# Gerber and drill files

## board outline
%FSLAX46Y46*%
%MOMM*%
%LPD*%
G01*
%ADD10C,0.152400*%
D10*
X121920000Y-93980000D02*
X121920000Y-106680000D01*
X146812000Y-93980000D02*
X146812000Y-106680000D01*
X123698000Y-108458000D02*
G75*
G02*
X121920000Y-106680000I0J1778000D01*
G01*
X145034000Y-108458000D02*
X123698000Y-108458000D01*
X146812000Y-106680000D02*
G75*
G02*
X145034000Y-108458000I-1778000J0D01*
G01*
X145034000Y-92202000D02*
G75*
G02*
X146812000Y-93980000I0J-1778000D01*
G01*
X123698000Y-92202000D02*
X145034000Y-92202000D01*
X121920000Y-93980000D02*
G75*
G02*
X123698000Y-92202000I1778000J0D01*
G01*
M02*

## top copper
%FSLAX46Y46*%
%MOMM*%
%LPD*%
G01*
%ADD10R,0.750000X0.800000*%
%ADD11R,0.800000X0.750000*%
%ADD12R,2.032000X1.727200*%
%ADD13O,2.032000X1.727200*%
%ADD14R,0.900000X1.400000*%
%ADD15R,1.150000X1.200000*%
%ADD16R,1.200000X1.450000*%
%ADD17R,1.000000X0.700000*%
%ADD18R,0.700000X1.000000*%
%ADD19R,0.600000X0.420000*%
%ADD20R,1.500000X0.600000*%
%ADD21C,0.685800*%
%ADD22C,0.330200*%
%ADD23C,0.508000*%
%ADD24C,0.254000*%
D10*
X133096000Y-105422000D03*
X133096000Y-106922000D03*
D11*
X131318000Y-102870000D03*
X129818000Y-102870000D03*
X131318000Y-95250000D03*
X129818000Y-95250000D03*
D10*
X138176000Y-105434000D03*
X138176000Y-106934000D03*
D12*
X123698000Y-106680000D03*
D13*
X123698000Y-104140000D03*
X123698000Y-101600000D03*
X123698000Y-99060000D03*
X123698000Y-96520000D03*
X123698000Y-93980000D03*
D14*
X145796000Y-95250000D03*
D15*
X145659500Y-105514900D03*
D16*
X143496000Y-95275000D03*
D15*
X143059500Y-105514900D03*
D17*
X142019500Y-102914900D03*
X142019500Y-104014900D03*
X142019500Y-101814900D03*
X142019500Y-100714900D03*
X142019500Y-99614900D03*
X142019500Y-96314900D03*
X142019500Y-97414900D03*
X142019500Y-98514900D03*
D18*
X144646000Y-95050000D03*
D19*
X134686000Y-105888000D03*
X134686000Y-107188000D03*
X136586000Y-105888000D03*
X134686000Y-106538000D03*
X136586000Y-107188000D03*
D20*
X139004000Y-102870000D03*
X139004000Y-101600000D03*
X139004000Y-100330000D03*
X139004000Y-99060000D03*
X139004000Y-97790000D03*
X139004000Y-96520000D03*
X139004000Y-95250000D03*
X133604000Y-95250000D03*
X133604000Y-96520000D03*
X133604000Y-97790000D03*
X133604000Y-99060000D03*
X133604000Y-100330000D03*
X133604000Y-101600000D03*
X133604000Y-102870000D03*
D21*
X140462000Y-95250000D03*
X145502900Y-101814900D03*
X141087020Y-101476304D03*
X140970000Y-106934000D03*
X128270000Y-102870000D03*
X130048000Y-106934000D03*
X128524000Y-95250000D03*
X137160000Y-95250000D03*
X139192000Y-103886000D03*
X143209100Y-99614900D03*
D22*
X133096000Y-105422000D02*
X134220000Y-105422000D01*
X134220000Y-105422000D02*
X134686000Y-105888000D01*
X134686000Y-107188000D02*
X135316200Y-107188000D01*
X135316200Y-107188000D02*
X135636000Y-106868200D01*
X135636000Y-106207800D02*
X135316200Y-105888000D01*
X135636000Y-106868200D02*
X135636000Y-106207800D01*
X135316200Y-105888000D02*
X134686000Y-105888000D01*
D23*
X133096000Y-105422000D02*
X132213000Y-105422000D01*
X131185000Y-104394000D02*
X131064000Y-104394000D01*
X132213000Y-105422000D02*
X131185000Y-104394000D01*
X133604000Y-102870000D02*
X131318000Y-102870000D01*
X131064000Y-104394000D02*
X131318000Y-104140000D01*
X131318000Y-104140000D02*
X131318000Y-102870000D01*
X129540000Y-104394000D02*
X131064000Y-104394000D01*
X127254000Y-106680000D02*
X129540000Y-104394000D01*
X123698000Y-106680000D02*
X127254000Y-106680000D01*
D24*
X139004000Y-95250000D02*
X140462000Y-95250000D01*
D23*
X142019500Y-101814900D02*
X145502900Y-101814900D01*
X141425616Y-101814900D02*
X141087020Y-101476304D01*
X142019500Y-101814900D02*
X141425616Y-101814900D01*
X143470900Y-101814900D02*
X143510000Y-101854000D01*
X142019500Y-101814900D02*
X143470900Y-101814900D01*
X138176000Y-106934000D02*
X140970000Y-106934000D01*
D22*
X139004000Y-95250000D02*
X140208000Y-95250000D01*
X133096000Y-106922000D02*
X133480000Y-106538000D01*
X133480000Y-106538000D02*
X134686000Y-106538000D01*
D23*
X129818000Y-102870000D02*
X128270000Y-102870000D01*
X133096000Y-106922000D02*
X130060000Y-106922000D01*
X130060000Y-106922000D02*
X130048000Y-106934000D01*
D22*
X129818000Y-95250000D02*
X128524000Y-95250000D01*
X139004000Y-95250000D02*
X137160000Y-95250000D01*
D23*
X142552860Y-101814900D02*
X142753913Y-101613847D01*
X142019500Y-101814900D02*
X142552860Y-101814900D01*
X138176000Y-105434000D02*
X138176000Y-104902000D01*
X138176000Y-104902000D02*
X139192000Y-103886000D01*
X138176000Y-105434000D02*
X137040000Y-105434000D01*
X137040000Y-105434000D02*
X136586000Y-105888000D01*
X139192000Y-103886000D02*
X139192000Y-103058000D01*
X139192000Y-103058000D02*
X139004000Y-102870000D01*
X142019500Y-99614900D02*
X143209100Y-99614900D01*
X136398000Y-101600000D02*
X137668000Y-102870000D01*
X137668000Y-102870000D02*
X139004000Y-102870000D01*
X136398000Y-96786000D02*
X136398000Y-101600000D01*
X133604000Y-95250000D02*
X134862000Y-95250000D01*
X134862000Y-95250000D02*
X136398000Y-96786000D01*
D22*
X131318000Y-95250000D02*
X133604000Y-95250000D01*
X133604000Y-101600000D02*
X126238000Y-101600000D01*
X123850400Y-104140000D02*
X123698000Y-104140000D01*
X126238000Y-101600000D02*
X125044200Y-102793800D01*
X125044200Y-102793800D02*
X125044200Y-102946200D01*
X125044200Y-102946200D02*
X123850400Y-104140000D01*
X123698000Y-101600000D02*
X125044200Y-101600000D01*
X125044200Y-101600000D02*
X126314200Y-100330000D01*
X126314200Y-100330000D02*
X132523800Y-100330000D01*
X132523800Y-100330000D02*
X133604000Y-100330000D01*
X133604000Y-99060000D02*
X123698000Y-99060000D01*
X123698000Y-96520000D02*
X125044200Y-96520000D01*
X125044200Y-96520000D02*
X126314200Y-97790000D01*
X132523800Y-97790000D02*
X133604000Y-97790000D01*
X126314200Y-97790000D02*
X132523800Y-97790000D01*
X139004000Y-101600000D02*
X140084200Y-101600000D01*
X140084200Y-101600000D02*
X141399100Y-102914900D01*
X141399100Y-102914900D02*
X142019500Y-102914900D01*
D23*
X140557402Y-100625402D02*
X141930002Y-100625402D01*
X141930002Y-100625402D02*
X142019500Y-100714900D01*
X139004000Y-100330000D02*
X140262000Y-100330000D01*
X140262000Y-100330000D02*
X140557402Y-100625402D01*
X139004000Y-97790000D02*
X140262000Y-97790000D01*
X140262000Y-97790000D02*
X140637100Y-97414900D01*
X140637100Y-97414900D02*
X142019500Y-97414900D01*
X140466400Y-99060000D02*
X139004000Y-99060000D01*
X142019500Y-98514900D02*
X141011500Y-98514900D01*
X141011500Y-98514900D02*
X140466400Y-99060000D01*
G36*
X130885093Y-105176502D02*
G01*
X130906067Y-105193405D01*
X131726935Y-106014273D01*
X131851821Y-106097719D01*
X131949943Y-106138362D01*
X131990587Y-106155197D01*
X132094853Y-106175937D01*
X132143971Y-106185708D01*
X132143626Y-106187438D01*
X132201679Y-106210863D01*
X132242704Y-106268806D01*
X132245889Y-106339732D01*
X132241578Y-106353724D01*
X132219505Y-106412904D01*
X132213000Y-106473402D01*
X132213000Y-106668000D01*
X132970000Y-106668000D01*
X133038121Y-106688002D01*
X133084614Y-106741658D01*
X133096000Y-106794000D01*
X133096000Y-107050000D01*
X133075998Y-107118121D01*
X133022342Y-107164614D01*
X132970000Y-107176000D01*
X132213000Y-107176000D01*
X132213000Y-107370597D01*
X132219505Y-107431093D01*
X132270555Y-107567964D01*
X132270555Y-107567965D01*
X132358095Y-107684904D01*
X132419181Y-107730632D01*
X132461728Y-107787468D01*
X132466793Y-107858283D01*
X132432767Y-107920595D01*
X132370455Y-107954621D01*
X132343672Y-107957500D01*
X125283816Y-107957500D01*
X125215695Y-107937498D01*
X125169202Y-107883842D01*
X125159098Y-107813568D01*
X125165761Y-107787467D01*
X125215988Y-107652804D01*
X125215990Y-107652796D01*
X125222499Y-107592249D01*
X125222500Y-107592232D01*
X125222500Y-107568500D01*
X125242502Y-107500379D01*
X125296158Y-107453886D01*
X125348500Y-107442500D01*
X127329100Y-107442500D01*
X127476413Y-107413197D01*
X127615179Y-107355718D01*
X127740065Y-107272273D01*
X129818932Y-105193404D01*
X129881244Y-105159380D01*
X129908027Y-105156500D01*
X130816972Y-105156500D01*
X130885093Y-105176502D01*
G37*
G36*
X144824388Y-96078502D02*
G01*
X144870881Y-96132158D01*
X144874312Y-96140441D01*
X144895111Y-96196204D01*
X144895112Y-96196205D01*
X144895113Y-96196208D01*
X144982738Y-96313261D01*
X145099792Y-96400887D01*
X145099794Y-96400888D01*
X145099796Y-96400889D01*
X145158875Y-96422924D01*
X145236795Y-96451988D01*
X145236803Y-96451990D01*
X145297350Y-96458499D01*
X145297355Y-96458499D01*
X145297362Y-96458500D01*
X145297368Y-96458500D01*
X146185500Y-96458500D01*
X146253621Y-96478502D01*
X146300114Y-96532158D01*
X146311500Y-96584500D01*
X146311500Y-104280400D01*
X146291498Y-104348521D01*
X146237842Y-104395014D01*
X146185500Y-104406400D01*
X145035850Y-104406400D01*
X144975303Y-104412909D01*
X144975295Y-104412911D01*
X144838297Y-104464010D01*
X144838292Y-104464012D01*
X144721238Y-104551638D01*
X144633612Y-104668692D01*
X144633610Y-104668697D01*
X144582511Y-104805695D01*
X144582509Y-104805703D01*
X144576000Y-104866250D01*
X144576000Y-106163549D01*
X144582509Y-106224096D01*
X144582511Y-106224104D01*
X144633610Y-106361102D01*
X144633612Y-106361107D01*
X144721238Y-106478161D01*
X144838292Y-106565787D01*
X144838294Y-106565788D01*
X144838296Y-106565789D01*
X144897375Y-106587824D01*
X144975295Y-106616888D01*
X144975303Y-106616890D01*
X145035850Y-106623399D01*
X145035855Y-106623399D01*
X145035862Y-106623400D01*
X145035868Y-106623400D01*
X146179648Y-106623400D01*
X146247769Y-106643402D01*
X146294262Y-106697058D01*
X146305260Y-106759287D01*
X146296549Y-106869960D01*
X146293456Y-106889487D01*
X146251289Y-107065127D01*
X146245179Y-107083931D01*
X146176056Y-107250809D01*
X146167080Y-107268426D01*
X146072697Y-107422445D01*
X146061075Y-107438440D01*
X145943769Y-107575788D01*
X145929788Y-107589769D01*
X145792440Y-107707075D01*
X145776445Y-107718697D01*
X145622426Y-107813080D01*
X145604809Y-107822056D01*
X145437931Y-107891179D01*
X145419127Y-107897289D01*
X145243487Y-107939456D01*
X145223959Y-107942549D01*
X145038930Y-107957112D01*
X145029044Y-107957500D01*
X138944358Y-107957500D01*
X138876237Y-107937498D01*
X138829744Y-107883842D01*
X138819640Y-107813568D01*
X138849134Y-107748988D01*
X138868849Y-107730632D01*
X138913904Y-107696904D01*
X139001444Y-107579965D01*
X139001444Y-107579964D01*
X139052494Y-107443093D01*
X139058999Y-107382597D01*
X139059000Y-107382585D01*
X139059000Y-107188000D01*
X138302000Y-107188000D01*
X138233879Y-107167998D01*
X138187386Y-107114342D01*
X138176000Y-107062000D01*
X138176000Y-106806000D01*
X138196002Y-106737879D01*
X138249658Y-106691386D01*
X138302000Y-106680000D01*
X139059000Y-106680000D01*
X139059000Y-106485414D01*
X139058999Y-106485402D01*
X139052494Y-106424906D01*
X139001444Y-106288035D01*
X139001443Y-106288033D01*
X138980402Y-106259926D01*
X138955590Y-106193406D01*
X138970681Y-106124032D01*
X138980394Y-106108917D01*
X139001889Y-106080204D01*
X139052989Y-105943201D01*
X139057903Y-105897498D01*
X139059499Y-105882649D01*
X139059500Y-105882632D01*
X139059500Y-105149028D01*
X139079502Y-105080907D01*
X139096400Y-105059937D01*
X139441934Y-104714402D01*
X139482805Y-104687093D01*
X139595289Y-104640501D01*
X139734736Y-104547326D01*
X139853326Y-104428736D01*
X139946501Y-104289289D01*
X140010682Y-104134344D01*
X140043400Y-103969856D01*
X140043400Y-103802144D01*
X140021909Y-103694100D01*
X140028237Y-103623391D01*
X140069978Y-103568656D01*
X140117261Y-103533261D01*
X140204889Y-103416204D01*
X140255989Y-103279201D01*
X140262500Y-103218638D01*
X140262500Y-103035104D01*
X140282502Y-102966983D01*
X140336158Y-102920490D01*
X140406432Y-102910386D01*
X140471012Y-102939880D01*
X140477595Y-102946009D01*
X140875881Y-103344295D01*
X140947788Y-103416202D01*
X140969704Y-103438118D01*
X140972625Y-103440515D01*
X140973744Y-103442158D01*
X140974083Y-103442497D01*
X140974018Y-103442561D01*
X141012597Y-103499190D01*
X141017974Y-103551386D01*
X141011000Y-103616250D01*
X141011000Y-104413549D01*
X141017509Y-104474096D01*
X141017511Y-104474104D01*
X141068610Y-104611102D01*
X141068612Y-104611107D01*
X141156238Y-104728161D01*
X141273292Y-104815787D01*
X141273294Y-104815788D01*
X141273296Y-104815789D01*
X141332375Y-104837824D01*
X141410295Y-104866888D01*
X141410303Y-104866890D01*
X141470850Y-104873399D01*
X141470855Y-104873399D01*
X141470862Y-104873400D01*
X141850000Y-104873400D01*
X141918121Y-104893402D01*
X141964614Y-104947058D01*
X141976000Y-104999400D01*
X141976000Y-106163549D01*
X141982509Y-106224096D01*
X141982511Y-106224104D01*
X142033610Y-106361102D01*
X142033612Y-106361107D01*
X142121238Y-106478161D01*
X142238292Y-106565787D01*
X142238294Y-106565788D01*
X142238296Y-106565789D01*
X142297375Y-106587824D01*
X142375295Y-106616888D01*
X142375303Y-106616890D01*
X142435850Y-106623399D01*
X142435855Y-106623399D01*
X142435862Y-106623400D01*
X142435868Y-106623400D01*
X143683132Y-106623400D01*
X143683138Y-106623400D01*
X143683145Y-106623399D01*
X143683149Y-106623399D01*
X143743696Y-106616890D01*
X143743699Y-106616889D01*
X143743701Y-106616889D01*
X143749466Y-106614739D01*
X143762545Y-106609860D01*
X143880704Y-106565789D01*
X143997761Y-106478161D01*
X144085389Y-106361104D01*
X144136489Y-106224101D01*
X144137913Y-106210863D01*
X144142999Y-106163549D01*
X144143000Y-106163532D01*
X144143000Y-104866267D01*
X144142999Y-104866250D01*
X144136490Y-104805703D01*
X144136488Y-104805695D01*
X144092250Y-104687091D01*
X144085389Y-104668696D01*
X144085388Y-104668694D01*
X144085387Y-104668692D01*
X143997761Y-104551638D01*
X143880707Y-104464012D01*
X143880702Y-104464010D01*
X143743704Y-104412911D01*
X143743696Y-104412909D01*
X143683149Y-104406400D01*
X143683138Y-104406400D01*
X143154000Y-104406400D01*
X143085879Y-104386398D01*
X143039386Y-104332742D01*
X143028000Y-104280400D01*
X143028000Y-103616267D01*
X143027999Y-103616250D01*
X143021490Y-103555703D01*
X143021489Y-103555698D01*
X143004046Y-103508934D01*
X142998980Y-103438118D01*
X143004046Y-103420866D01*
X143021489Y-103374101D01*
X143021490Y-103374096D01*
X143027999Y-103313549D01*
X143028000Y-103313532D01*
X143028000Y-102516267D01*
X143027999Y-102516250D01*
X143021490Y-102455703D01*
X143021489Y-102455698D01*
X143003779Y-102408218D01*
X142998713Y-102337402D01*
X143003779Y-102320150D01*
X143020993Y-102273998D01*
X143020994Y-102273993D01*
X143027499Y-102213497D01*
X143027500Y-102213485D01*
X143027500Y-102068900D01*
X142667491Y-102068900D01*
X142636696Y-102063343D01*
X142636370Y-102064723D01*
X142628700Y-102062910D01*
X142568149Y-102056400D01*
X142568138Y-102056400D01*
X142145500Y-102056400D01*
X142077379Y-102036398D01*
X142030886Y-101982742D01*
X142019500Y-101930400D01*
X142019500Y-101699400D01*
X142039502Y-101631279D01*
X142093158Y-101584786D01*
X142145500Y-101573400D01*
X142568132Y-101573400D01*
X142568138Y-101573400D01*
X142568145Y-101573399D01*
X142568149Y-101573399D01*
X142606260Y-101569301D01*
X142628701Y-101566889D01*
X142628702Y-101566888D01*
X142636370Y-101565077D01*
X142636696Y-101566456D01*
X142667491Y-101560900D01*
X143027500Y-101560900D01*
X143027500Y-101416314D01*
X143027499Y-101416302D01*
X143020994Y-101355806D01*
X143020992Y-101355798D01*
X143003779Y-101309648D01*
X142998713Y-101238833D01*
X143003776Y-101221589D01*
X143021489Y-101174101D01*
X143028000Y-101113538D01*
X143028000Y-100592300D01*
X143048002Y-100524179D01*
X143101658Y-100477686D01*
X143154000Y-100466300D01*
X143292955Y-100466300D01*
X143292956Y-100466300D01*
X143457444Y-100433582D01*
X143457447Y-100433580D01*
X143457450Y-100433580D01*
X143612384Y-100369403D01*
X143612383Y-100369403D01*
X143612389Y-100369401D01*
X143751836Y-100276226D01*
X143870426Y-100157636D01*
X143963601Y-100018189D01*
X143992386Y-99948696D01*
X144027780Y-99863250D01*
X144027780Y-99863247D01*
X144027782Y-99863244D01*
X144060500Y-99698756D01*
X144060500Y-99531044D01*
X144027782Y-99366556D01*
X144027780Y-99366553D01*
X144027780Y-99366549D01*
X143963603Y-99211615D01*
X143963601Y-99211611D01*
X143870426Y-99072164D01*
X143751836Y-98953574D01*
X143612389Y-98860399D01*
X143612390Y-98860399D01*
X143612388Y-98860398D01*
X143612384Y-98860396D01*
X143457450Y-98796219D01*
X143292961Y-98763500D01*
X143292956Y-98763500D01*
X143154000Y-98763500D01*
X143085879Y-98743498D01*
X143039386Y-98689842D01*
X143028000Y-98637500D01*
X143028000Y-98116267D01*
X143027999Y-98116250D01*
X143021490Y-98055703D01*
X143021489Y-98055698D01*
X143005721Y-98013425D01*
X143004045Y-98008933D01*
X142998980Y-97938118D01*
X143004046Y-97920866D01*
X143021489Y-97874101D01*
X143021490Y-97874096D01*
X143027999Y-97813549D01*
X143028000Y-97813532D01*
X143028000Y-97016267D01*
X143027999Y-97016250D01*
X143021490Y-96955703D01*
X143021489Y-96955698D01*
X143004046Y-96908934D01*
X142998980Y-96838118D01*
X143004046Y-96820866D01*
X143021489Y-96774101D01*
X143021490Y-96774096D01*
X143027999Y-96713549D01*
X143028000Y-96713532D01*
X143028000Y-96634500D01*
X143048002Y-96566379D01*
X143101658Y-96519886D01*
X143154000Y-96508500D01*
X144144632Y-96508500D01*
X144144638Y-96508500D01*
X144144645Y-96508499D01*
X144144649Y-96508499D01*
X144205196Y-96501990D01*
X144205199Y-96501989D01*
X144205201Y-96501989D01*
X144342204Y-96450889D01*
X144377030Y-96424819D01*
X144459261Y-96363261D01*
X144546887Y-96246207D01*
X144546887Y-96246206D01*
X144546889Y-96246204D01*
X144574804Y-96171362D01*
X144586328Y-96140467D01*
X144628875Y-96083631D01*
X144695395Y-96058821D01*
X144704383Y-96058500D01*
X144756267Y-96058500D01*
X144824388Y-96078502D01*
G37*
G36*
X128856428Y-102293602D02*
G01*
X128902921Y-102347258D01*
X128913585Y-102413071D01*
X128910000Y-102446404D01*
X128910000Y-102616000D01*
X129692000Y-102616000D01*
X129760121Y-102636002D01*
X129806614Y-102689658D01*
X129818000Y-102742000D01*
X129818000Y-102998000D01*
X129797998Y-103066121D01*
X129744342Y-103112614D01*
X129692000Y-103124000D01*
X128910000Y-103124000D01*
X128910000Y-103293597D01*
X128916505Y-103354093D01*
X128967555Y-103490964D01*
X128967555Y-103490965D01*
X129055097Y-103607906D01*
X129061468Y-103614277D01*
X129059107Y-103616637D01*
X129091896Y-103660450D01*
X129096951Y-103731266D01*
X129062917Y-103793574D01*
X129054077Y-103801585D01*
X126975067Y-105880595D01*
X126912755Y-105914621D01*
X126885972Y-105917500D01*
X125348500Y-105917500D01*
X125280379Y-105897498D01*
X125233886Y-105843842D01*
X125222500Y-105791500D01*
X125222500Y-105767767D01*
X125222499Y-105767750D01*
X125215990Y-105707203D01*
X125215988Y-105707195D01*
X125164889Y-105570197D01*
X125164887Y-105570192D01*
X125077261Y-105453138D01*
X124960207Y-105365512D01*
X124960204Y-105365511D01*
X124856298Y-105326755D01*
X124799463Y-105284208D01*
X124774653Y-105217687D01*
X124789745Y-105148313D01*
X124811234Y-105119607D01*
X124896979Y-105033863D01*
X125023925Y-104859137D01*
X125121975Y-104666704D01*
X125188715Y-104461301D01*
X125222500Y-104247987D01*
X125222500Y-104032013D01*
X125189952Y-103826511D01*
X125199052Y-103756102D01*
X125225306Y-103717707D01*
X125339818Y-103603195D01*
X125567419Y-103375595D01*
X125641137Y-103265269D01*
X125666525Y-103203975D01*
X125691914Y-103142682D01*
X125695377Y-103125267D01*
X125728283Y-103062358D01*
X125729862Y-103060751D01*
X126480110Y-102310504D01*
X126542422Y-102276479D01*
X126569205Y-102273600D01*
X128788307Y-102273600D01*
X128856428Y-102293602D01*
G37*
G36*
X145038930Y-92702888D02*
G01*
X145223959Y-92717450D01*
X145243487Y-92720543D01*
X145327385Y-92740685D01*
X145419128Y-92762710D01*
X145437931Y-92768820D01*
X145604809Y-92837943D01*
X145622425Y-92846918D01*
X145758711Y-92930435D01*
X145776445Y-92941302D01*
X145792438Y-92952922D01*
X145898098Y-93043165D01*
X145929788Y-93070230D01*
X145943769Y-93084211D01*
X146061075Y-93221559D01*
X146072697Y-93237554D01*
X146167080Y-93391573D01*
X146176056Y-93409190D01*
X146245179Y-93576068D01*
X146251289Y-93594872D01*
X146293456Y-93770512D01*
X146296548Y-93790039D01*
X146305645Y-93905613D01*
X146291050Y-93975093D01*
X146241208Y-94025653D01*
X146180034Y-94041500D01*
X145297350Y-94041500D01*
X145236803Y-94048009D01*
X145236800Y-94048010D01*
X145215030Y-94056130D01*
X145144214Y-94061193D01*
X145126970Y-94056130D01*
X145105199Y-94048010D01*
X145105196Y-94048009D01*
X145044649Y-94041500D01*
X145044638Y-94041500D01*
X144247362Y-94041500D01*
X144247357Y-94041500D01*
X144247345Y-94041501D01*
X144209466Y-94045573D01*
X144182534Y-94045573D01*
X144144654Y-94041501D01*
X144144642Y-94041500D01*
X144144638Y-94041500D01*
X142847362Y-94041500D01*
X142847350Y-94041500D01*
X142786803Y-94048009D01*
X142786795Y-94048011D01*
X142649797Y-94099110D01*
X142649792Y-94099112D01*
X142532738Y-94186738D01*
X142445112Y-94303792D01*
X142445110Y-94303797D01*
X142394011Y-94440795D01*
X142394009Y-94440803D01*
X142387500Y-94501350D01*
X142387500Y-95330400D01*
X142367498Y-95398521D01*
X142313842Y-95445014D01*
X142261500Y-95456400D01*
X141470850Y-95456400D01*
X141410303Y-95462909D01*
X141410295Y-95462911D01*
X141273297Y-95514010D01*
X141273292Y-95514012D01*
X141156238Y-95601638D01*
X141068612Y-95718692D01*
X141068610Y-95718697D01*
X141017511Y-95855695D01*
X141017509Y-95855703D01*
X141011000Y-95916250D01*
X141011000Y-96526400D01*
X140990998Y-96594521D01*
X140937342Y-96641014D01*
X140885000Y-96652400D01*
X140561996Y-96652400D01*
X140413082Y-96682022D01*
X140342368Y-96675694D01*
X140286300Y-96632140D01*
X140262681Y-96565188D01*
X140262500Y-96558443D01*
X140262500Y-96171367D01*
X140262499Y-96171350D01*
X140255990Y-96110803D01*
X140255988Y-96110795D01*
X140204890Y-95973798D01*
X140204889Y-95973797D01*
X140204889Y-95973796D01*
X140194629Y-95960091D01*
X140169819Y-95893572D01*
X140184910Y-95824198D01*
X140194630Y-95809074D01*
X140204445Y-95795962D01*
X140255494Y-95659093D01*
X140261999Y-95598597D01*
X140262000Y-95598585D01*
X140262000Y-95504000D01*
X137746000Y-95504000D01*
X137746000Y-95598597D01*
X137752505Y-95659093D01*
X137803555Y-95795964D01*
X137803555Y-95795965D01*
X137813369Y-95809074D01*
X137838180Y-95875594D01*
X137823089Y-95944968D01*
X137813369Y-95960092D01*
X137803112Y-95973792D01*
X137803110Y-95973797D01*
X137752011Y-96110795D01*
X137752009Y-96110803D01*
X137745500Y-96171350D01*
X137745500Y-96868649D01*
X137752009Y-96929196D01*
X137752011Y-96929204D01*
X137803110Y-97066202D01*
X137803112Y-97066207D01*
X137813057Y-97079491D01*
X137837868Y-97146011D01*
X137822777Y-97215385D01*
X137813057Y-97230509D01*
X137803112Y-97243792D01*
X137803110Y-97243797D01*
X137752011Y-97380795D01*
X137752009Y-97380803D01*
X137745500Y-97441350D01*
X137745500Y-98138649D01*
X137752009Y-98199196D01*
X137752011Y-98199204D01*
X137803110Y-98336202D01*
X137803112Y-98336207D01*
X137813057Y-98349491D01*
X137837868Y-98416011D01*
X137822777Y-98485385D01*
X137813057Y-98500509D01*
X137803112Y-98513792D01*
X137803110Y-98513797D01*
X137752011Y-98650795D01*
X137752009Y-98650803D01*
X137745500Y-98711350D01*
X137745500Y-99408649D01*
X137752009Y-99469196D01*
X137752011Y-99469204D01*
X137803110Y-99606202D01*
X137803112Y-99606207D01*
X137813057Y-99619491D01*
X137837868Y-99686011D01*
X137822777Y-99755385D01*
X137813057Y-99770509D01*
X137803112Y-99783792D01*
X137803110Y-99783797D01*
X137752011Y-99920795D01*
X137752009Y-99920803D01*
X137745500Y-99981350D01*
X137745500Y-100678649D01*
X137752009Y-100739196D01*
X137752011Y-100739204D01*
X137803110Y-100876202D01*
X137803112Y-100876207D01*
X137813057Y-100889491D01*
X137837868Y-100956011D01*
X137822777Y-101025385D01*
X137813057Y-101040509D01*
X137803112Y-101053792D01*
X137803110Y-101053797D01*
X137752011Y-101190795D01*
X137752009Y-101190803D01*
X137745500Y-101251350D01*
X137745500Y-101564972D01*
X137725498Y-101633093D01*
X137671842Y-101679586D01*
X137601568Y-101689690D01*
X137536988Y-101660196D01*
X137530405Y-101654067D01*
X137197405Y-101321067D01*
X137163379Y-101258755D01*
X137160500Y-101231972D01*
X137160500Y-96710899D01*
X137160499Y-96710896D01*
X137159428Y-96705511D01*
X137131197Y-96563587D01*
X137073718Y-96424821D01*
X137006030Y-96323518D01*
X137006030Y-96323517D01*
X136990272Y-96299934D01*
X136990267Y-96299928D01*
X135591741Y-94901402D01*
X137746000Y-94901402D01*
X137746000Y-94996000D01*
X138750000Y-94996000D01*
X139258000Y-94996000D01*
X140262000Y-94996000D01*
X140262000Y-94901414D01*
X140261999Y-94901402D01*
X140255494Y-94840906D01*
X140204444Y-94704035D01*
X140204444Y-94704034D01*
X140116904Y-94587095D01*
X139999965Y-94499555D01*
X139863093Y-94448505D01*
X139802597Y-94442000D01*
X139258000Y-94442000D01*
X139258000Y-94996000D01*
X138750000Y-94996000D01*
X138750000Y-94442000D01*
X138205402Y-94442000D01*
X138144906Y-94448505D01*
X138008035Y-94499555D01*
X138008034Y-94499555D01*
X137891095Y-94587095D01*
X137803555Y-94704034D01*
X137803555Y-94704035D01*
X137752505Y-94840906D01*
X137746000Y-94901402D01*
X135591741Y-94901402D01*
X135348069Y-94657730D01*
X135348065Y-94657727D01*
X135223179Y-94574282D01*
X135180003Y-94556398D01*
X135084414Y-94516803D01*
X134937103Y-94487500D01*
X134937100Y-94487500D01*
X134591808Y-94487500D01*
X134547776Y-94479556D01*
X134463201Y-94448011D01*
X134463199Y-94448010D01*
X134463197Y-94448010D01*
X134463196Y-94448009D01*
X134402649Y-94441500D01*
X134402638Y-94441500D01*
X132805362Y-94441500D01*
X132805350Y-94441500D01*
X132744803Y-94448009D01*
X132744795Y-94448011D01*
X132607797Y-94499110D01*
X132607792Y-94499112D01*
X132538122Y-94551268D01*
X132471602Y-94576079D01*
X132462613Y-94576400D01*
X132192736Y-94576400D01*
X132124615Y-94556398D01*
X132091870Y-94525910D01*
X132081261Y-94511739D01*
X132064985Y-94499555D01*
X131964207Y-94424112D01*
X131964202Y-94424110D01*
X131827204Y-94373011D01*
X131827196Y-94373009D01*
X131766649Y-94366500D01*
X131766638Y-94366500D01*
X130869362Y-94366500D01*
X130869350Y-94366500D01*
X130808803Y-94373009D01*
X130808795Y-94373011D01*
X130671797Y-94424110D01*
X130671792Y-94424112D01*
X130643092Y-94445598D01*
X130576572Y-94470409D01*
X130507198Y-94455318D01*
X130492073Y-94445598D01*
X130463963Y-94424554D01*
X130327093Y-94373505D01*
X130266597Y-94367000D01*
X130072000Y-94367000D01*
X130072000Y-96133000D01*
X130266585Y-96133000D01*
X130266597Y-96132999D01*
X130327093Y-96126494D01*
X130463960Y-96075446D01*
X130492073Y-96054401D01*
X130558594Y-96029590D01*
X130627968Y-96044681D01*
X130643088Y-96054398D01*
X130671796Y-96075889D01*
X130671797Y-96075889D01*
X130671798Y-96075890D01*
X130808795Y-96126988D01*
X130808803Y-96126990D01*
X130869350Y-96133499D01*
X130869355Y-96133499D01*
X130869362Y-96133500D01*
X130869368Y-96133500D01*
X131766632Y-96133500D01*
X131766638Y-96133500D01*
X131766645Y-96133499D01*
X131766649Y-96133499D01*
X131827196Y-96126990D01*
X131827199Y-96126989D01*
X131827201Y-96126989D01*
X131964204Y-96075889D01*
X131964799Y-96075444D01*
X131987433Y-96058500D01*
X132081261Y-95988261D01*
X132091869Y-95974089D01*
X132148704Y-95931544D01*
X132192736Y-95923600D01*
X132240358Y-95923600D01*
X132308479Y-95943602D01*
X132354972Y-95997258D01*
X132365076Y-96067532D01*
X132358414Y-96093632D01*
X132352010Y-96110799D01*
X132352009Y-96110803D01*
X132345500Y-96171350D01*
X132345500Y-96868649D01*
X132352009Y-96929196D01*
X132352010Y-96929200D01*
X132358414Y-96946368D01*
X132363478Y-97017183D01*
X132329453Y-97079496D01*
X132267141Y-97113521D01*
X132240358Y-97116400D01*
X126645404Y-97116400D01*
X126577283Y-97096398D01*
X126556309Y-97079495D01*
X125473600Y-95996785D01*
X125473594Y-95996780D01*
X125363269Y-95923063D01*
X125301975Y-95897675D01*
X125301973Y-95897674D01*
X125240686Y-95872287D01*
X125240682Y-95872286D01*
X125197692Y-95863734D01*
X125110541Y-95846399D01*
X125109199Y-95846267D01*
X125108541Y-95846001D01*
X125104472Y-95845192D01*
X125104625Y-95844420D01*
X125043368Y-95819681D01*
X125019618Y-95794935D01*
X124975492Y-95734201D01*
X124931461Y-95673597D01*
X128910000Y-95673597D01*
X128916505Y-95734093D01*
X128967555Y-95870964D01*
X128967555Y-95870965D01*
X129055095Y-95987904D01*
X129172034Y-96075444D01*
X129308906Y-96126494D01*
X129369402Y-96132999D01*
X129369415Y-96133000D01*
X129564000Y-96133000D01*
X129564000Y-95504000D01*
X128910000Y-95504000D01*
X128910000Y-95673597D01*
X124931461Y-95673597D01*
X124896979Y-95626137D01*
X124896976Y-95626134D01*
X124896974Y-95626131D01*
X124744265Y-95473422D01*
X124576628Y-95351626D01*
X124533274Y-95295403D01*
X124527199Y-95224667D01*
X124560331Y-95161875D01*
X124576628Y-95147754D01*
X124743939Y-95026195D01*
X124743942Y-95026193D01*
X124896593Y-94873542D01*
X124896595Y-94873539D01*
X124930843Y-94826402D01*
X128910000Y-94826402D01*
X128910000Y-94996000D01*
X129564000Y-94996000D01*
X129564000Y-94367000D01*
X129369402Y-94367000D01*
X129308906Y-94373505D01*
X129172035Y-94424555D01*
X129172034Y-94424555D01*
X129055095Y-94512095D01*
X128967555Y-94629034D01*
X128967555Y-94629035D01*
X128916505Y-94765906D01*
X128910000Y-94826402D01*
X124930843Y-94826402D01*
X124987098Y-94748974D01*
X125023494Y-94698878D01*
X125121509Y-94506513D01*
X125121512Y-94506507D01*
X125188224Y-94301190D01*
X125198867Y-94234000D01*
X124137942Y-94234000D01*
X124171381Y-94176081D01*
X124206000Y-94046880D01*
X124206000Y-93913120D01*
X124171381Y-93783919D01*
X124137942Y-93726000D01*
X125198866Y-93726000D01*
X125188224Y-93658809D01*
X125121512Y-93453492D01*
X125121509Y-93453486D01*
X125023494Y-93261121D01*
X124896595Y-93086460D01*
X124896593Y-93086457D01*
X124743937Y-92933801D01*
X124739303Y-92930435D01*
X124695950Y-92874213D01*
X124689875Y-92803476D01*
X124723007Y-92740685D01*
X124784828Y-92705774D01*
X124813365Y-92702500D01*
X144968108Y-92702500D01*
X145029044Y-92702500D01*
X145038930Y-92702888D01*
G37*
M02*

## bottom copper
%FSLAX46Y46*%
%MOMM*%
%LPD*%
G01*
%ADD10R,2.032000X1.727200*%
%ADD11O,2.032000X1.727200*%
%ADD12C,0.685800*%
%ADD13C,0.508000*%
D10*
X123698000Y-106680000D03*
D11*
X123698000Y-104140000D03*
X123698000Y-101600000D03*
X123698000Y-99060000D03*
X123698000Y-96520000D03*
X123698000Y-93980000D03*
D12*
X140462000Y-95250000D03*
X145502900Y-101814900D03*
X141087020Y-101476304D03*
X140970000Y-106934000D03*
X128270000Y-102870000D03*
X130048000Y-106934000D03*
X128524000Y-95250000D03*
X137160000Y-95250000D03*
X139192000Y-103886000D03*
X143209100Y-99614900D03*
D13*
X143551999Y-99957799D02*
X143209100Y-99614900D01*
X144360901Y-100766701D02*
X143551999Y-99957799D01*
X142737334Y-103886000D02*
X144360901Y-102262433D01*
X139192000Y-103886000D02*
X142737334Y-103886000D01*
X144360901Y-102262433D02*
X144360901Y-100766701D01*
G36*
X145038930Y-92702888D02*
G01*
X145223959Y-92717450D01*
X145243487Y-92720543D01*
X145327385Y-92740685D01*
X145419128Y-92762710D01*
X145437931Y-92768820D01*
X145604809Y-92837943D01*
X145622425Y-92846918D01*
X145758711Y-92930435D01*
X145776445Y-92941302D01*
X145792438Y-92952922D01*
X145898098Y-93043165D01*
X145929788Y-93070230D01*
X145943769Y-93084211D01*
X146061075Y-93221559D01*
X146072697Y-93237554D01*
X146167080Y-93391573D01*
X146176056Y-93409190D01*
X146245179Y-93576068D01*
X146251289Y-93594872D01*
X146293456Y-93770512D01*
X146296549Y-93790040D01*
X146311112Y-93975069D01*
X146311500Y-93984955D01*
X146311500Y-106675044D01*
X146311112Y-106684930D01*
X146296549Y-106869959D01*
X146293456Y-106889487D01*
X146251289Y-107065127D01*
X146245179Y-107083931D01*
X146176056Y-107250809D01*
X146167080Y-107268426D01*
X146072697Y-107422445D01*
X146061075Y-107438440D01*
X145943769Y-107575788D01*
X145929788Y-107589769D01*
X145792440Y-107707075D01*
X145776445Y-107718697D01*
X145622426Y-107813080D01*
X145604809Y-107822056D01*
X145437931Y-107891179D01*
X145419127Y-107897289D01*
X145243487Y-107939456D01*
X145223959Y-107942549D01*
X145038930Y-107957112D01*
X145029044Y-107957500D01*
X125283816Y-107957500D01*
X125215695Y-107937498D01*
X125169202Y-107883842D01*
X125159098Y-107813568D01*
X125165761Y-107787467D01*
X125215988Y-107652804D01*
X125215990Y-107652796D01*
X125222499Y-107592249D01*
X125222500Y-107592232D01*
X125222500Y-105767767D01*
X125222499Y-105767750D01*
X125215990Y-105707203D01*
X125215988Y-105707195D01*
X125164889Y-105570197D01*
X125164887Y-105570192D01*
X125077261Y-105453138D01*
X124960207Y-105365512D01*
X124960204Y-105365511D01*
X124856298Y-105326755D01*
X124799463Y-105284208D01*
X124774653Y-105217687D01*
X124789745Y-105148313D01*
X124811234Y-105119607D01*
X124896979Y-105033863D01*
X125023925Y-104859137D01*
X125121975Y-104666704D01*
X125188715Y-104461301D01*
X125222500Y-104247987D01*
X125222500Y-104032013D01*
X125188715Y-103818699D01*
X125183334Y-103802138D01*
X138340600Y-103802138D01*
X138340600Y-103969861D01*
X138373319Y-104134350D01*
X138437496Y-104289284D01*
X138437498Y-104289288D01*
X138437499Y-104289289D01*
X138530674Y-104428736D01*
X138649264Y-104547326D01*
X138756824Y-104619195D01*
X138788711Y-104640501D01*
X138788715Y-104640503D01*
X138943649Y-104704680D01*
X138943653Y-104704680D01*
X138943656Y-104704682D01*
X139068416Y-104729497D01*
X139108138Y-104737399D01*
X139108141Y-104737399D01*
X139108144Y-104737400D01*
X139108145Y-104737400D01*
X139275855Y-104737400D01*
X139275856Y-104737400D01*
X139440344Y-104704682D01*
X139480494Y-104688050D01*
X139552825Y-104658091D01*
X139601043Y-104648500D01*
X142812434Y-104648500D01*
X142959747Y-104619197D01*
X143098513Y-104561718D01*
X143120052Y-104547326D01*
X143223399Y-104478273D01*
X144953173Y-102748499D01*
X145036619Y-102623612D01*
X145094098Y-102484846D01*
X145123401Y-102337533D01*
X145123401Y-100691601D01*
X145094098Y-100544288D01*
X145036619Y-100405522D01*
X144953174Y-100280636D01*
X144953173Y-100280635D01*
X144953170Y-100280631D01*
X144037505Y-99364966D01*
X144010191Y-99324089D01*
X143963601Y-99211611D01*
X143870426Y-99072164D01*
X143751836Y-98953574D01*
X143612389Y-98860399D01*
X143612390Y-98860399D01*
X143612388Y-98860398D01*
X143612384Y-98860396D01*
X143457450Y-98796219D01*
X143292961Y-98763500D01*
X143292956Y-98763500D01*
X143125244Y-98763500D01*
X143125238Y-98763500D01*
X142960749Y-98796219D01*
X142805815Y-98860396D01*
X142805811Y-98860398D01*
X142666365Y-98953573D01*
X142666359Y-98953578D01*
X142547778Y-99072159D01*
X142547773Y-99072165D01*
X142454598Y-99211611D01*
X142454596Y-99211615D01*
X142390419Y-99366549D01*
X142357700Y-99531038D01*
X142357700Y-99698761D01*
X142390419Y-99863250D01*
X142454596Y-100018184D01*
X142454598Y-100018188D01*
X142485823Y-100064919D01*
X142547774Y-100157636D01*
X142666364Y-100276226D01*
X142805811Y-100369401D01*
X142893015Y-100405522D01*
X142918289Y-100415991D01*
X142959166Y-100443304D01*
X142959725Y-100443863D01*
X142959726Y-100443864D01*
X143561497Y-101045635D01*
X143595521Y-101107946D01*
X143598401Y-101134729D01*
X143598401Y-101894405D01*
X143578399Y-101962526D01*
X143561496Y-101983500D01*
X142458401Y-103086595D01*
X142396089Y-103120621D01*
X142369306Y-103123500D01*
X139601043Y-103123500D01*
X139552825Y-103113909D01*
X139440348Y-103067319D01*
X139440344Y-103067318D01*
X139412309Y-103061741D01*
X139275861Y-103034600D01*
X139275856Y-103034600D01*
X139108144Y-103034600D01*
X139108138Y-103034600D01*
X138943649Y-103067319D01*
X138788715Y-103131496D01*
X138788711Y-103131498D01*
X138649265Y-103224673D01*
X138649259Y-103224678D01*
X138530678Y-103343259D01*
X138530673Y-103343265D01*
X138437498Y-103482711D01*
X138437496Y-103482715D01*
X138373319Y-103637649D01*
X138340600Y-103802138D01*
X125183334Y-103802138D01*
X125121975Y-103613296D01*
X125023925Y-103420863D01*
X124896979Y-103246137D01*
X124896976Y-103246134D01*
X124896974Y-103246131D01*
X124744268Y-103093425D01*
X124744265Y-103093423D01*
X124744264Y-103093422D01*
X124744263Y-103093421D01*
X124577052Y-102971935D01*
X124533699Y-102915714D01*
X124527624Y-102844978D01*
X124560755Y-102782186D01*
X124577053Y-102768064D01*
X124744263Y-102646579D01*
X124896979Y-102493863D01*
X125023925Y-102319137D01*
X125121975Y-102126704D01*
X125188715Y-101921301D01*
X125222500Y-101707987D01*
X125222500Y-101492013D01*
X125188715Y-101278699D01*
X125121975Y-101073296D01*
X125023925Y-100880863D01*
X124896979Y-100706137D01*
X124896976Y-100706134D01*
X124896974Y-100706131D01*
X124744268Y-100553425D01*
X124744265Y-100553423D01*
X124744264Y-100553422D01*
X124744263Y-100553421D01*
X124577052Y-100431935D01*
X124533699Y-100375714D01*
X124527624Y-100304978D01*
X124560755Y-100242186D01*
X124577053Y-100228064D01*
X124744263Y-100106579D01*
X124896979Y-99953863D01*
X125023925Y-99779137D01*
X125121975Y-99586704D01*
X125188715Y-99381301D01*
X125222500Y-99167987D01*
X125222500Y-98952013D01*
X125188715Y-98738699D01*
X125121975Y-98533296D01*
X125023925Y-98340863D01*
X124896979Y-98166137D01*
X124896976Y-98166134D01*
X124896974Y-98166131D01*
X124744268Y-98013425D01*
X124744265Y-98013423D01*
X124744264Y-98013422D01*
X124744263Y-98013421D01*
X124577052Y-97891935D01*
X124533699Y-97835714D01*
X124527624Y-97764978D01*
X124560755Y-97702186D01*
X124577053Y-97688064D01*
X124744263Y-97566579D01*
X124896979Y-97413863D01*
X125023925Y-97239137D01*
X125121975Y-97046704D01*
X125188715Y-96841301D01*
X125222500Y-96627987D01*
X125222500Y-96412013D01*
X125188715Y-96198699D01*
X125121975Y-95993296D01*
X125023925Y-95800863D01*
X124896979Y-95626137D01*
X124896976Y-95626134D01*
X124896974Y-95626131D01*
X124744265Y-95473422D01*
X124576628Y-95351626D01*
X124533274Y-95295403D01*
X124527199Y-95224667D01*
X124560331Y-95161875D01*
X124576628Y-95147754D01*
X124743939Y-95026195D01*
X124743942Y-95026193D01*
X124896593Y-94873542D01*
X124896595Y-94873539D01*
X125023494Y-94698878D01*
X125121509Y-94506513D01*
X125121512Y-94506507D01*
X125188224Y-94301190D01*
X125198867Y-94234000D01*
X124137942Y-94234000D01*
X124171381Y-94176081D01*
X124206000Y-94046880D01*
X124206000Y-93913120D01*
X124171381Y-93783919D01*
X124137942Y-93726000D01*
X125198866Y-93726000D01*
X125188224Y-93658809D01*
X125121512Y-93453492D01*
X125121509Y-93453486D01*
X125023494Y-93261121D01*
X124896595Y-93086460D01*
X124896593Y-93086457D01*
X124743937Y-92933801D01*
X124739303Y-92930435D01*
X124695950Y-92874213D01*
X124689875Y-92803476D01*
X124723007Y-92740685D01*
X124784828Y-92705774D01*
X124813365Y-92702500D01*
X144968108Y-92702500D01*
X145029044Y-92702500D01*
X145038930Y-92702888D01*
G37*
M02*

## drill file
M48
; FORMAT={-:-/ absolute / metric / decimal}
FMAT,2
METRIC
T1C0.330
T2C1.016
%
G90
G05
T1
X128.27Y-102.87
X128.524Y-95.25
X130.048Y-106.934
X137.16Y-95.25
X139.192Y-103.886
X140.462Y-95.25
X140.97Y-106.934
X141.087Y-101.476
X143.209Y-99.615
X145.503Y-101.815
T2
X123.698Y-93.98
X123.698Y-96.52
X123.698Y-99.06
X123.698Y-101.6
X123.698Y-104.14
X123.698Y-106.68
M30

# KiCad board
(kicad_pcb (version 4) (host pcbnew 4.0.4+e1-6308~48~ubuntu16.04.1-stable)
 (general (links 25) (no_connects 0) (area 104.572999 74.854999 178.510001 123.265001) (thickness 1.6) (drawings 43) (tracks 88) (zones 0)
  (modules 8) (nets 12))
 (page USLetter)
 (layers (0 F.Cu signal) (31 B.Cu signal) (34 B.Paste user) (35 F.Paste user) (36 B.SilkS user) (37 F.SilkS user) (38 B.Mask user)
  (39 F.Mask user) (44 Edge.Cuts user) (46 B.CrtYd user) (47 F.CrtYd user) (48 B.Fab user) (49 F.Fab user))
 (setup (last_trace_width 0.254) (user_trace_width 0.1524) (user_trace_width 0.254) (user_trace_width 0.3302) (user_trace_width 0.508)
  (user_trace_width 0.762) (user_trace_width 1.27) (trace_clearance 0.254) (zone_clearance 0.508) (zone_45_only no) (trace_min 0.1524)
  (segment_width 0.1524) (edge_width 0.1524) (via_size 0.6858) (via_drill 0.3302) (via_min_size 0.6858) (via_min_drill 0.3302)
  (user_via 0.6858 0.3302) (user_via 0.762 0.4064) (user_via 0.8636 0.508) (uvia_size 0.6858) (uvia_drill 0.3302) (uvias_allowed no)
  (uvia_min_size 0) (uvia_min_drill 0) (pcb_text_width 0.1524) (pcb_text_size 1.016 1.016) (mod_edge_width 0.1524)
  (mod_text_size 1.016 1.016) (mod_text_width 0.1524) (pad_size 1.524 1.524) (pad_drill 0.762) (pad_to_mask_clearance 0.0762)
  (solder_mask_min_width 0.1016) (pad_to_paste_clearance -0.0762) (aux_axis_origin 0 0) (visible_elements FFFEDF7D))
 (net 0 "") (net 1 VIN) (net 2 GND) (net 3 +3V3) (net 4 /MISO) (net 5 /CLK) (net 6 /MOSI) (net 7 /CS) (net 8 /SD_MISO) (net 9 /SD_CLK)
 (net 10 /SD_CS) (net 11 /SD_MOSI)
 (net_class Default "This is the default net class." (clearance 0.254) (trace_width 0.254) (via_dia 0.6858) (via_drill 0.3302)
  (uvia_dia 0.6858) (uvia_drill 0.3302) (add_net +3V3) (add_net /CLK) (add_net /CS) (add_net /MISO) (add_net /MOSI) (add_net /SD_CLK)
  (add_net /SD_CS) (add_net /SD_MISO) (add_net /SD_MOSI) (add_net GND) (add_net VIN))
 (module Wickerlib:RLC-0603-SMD (layer F.Cu) (at 133.096 106.172 270)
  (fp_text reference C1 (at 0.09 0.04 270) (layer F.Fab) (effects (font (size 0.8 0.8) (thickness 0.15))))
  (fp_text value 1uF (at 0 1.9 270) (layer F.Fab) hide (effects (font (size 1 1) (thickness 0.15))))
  (pad 1 smd rect (at -0.75 0 270) (size 0.8 0.75) (layers F.Cu F.Paste F.Mask) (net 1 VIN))
  (pad 2 smd rect (at 0.75 0 270) (size 0.8 0.75) (layers F.Cu F.Paste F.Mask) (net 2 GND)))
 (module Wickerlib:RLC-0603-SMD (layer F.Cu) (at 130.568 102.87 180)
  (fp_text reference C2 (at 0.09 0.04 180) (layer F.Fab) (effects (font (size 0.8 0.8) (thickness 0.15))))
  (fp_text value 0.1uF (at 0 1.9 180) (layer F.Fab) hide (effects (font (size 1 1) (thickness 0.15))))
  (pad 1 smd rect (at -0.75 0 180) (size 0.8 0.75) (layers F.Cu F.Paste F.Mask) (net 1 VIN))
  (pad 2 smd rect (at 0.75 0 180) (size 0.8 0.75) (layers F.Cu F.Paste F.Mask) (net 2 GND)))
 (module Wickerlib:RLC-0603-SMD (layer F.Cu) (at 130.568 95.25 180)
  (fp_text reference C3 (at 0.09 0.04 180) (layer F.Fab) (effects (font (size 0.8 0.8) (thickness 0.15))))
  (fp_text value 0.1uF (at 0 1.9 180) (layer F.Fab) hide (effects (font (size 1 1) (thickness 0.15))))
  (pad 1 smd rect (at -0.75 0 180) (size 0.8 0.75) (layers F.Cu F.Paste F.Mask) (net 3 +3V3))
  (pad 2 smd rect (at 0.75 0 180) (size 0.8 0.75) (layers F.Cu F.Paste F.Mask) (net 2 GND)))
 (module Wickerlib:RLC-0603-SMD (layer F.Cu) (at 138.176 106.184 270)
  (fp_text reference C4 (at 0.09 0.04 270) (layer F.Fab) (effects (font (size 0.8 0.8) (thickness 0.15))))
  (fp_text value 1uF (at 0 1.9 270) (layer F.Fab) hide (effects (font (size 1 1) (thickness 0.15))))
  (pad 1 smd rect (at -0.75 0 270) (size 0.8 0.75) (layers F.Cu F.Paste F.Mask) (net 3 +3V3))
  (pad 2 smd rect (at 0.75 0 270) (size 0.8 0.75) (layers F.Cu F.Paste F.Mask) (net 2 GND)))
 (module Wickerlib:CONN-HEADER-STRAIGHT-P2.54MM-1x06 (layer F.Cu) (at 123.698 106.68 180)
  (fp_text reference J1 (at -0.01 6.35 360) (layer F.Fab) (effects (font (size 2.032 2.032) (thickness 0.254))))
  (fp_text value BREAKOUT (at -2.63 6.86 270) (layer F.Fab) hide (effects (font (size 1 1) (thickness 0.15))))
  (pad 1 thru_hole rect (at 0 0 180) (size 2.032 1.7272) (drill 1.016) (layers *.Cu *.Mask F.SilkS) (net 1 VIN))
  (pad 2 thru_hole oval (at 0 2.54 180) (size 2.032 1.7272) (drill 1.016) (layers *.Cu *.Mask F.SilkS) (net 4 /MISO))
  (pad 3 thru_hole oval (at 0 5.08 180) (size 2.032 1.7272) (drill 1.016) (layers *.Cu *.Mask F.SilkS) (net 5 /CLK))
  (pad 4 thru_hole oval (at 0 7.62 180) (size 2.032 1.7272) (drill 1.016) (layers *.Cu *.Mask F.SilkS) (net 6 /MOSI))
  (pad 5 thru_hole oval (at 0 10.16 180) (size 2.032 1.7272) (drill 1.016) (layers *.Cu *.Mask F.SilkS) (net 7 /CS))
  (pad 6 thru_hole oval (at 0 12.7 180) (size 2.032 1.7272) (drill 1.016) (layers *.Cu *.Mask F.SilkS) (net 2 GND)))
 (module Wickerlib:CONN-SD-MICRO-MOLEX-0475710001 (layer F.Cu) (at 140.696 100.1014 90)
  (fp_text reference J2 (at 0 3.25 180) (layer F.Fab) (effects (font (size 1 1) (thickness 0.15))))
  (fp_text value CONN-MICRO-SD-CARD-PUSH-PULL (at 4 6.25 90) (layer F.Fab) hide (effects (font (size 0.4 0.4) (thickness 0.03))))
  (pad G5 smd rect (at 4.8514 5.1 90) (size 1.4 0.9) (layers F.Cu F.Paste F.Mask))
  (pad G2 smd rect (at -5.4135 4.9635 90) (size 1.2 1.15) (layers F.Cu F.Paste F.Mask))
  (pad G3 smd rect (at 4.8264 2.8 90) (size 1.45 1.2) (layers F.Cu F.Paste F.Mask))
  (pad G1 smd rect (at -5.4135 2.3635 90) (size 1.2 1.15) (layers F.Cu F.Paste F.Mask))
  (pad 7 smd rect (at -2.8135 1.3235 90) (size 0.7 1) (layers F.Cu F.Paste F.Mask) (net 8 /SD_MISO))
  (pad 8 smd rect (at -3.9135 1.3235 90) (size 0.7 1) (layers F.Cu F.Paste F.Mask))
  (pad 6 smd rect (at -1.7135 1.3235 90) (size 0.7 1) (layers F.Cu F.Paste F.Mask) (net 2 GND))
  (pad 5 smd rect (at -0.6135 1.3235 90) (size 0.7 1) (layers F.Cu F.Paste F.Mask) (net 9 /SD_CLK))
  (pad 4 smd rect (at 0.4865 1.3235 90) (size 0.7 1) (layers F.Cu F.Paste F.Mask) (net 3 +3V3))
  (pad 1 smd rect (at 3.7865 1.3235 90) (size 0.7 1) (layers F.Cu F.Paste F.Mask))
  (pad 2 smd rect (at 2.6865 1.3235 90) (size 0.7 1) (layers F.Cu F.Paste F.Mask) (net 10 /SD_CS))
  (pad 3 smd rect (at 1.5865 1.3235 90) (size 0.7 1) (layers F.Cu F.Paste F.Mask) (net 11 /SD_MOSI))
  (pad G4 smd rect (at 5.0514 3.95 90) (size 1 0.7) (layers F.Cu F.Paste F.Mask)))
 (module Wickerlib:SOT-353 (layer F.Cu) (at 135.636 106.538)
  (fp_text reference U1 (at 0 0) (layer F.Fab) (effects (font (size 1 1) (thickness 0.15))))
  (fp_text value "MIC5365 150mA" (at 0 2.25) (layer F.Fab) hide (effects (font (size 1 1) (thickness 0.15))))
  (pad 1 smd rect (at -0.95 -0.65) (size 0.6 0.42) (layers F.Cu F.Paste F.Mask) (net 1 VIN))
  (pad 3 smd rect (at -0.95 0.65) (size 0.6 0.42) (layers F.Cu F.Paste F.Mask) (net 1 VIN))
  (pad 5 smd rect (at 0.95 -0.65) (size 0.6 0.42) (layers F.Cu F.Paste F.Mask) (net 3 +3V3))
  (pad 2 smd rect (at -0.95 0) (size 0.6 0.42) (layers F.Cu F.Paste F.Mask) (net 2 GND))
  (pad 4 smd rect (at 0.95 0.65) (size 0.6 0.42) (layers F.Cu F.Paste F.Mask)))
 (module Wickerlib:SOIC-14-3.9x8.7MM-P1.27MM (layer F.Cu) (at 136.304 99.06 180)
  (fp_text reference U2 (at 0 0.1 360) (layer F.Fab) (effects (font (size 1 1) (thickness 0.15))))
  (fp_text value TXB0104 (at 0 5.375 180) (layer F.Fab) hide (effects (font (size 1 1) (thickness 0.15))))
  (pad 1 smd rect (at -2.7 -3.81 180) (size 1.5 0.6) (layers F.Cu F.Paste F.Mask) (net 3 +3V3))
  (pad 2 smd rect (at -2.7 -2.54 180) (size 1.5 0.6) (layers F.Cu F.Paste F.Mask) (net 8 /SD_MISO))
  (pad 3 smd rect (at -2.7 -1.27 180) (size 1.5 0.6) (layers F.Cu F.Paste F.Mask) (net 9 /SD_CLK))
  (pad 4 smd rect (at -2.7 0 180) (size 1.5 0.6) (layers F.Cu F.Paste F.Mask) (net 11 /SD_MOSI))
  (pad 5 smd rect (at -2.7 1.27 180) (size 1.5 0.6) (layers F.Cu F.Paste F.Mask) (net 10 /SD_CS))
  (pad 6 smd rect (at -2.7 2.54 180) (size 1.5 0.6) (layers F.Cu F.Paste F.Mask))
  (pad 7 smd rect (at -2.7 3.81 180) (size 1.5 0.6) (layers F.Cu F.Paste F.Mask) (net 2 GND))
  (pad 8 smd rect (at 2.7 3.81 180) (size 1.5 0.6) (layers F.Cu F.Paste F.Mask) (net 3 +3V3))
  (pad 9 smd rect (at 2.7 2.54 180) (size 1.5 0.6) (layers F.Cu F.Paste F.Mask))
  (pad 10 smd rect (at 2.7 1.27 180) (size 1.5 0.6) (layers F.Cu F.Paste F.Mask) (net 7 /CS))
  (pad 11 smd rect (at 2.7 0 180) (size 1.5 0.6) (layers F.Cu F.Paste F.Mask) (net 6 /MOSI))
  (pad 12 smd rect (at 2.7 -1.27 180) (size 1.5 0.6) (layers F.Cu F.Paste F.Mask) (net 5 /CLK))
  (pad 13 smd rect (at 2.7 -2.54 180) (size 1.5 0.6) (layers F.Cu F.Paste F.Mask) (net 4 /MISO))
  (pad 14 smd rect (at 2.7 -3.81 180) (size 1.5 0.6) (layers F.Cu F.Paste F.Mask) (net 1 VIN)))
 (gr_line (start 121.92 93.98) (end 121.92 106.68) (layer Edge.Cuts) (width 0.1524))
 (gr_line (start 146.812 93.98) (end 146.812 106.68) (layer Edge.Cuts) (width 0.1524))
 (gr_arc (start 123.698 106.68) (end 123.698 108.458) (angle 90) (layer Edge.Cuts) (width 0.1524))
 (gr_line (start 145.034 108.458) (end 123.698 108.458) (layer Edge.Cuts) (width 0.1524))
 (gr_arc (start 145.034 106.68) (end 146.812 106.68) (angle 90) (layer Edge.Cuts) (width 0.1524))
 (gr_arc (start 145.034 93.98) (end 145.034 92.202) (angle 90) (layer Edge.Cuts) (width 0.1524))
 (gr_line (start 123.698 92.202) (end 145.034 92.202) (layer Edge.Cuts) (width 0.1524))
 (gr_arc (start 123.698 93.98) (end 121.92 93.98) (angle 90) (layer Edge.Cuts) (width 0.1524))
 (segment (start 133.096 105.422) (end 134.22 105.422) (width 0.3302) (layer F.Cu) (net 1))
 (segment (start 134.22 105.422) (end 134.686 105.888) (width 0.3302) (layer F.Cu) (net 1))
 (segment (start 134.686 107.188) (end 135.3162 107.188) (width 0.3302) (layer F.Cu) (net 1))
 (segment (start 135.3162 107.188) (end 135.636 106.8682) (width 0.3302) (layer F.Cu) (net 1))
 (segment (start 135.636 106.2078) (end 135.3162 105.888) (width 0.3302) (layer F.Cu) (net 1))
 (segment (start 135.636 106.8682) (end 135.636 106.2078) (width 0.3302) (layer F.Cu) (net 1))
 (segment (start 135.3162 105.888) (end 134.686 105.888) (width 0.3302) (layer F.Cu) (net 1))
 (segment (start 133.096 105.422) (end 132.213 105.422) (width 0.508) (layer F.Cu) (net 1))
 (segment (start 131.185 104.394) (end 131.064 104.394) (width 0.508) (layer F.Cu) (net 1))
 (segment (start 132.213 105.422) (end 131.185 104.394) (width 0.508) (layer F.Cu) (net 1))
 (segment (start 133.604 102.87) (end 131.318 102.87) (width 0.508) (layer F.Cu) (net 1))
 (segment (start 131.064 104.394) (end 131.318 104.14) (width 0.508) (layer F.Cu) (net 1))
 (segment (start 131.318 104.14) (end 131.318 102.87) (width 0.508) (layer F.Cu) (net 1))
 (segment (start 129.54 104.394) (end 131.064 104.394) (width 0.508) (layer F.Cu) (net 1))
 (segment (start 127.254 106.68) (end 129.54 104.394) (width 0.508) (layer F.Cu) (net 1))
 (segment (start 123.698 106.68) (end 127.254 106.68) (width 0.508) (layer F.Cu) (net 1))
 (segment (start 139.004 95.25) (end 140.462 95.25) (width 0.254) (layer F.Cu) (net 2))
 (via (at 140.462 95.25) (size 0.6858) (drill 0.3302) (layers F.Cu B.Cu) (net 2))
 (via (at 145.5029 101.8149) (size 0.6858) (drill 0.3302) (layers F.Cu B.Cu) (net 2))
 (segment (start 142.0195 101.8149) (end 145.5029 101.8149) (width 0.508) (layer F.Cu) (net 2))
 (segment (start 141.425616 101.8149) (end 141.08702 101.476304) (width 0.508) (layer F.Cu) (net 2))
 (segment (start 142.0195 101.8149) (end 141.425616 101.8149) (width 0.508) (layer F.Cu) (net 2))
 (via (at 141.08702 101.476304) (size 0.6858) (drill 0.3302) (layers F.Cu B.Cu) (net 2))
 (segment (start 143.4709 101.8149) (end 143.51 101.854) (width 0.508) (layer F.Cu) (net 2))
 (segment (start 142.0195 101.8149) (end 143.4709 101.8149) (width 0.508) (layer F.Cu) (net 2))
 (segment (start 138.176 106.934) (end 140.97 106.934) (width 0.508) (layer F.Cu) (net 2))
 (via (at 140.97 106.934) (size 0.6858) (drill 0.3302) (layers F.Cu B.Cu) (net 2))
 (segment (start 139.004 95.25) (end 140.208 95.25) (width 0.3302) (layer F.Cu) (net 2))
 (segment (start 133.096 106.922) (end 133.48 106.538) (width 0.3302) (layer F.Cu) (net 2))
 (segment (start 133.48 106.538) (end 134.686 106.538) (width 0.3302) (layer F.Cu) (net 2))
 (segment (start 129.818 102.87) (end 128.27 102.87) (width 0.508) (layer F.Cu) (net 2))
 (via (at 128.27 102.87) (size 0.6858) (drill 0.3302) (layers F.Cu B.Cu) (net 2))
 (segment (start 133.096 106.922) (end 130.06 106.922) (width 0.508) (layer F.Cu) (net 2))
 (segment (start 130.06 106.922) (end 130.048 106.934) (width 0.508) (layer F.Cu) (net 2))
 (via (at 130.048 106.934) (size 0.6858) (drill 0.3302) (layers F.Cu B.Cu) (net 2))
 (segment (start 129.818 95.25) (end 128.524 95.25) (width 0.3302) (layer F.Cu) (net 2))
 (via (at 128.524 95.25) (size 0.6858) (drill 0.3302) (layers F.Cu B.Cu) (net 2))
 (segment (start 139.004 95.25) (end 137.16 95.25) (width 0.3302) (layer F.Cu) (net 2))
 (via (at 137.16 95.25) (size 0.6858) (drill 0.3302) (layers F.Cu B.Cu) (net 2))
 (segment (start 142.55286 101.8149) (end 142.753913 101.613847) (width 0.508) (layer F.Cu) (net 2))
 (segment (start 142.0195 101.8149) (end 142.55286 101.8149) (width 0.508) (layer F.Cu) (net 2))
 (segment (start 143.551999 99.957799) (end 143.2091 99.6149) (width 0.508) (layer B.Cu) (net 3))
 (segment (start 144.360901 100.766701) (end 143.551999 99.957799) (width 0.508) (layer B.Cu) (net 3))
 (segment (start 142.737334 103.886) (end 144.360901 102.262433) (width 0.508) (layer B.Cu) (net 3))
 (segment (start 139.192 103.886) (end 142.737334 103.886) (width 0.508) (layer B.Cu) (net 3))
 (segment (start 144.360901 102.262433) (end 144.360901 100.766701) (width 0.508) (layer B.Cu) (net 3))
 (segment (start 138.176 105.434) (end 138.176 104.902) (width 0.508) (layer F.Cu) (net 3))
 (segment (start 138.176 104.902) (end 139.192 103.886) (width 0.508) (layer F.Cu) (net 3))
 (segment (start 138.176 105.434) (end 137.04 105.434) (width 0.508) (layer F.Cu) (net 3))
 (segment (start 137.04 105.434) (end 136.586 105.888) (width 0.508) (layer F.Cu) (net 3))
 (segment (start 139.192 103.886) (end 139.192 103.058) (width 0.508) (layer F.Cu) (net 3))
 (segment (start 139.192 103.058) (end 139.004 102.87) (width 0.508) (layer F.Cu) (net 3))
 (via (at 139.192 103.886) (size 0.6858) (drill 0.3302) (layers F.Cu B.Cu) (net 3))
 (via (at 143.2091 99.6149) (size 0.6858) (drill 0.3302) (layers F.Cu B.Cu) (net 3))
 (segment (start 142.0195 99.6149) (end 143.2091 99.6149) (width 0.508) (layer F.Cu) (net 3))
 (segment (start 136.398 101.6) (end 137.668 102.87) (width 0.508) (layer F.Cu) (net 3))
 (segment (start 137.668 102.87) (end 139.004 102.87) (width 0.508) (layer F.Cu) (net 3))
 (segment (start 136.398 96.786) (end 136.398 101.6) (width 0.508) (layer F.Cu) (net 3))
 (segment (start 133.604 95.25) (end 134.862 95.25) (width 0.508) (layer F.Cu) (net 3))
 (segment (start 134.862 95.25) (end 136.398 96.786) (width 0.508) (layer F.Cu) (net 3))
 (segment (start 131.318 95.25) (end 133.604 95.25) (width 0.3302) (layer F.Cu) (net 3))
 (segment (start 133.604 101.6) (end 126.238 101.6) (width 0.3302) (layer F.Cu) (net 4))
 (segment (start 123.8504 104.14) (end 123.698 104.14) (width 0.3302) (layer F.Cu) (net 4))
 (segment (start 126.238 101.6) (end 125.0442 102.7938) (width 0.3302) (layer F.Cu) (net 4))
 (segment (start 125.0442 102.7938) (end 125.0442 102.9462) (width 0.3302) (layer F.Cu) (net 4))
 (segment (start 125.0442 102.9462) (end 123.8504 104.14) (width 0.3302) (layer F.Cu) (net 4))
 (segment (start 123.698 101.6) (end 125.0442 101.6) (width 0.3302) (layer F.Cu) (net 5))
 (segment (start 125.0442 101.6) (end 126.3142 100.33) (width 0.3302) (layer F.Cu) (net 5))
 (segment (start 126.3142 100.33) (end 132.5238 100.33) (width 0.3302) (layer F.Cu) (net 5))
 (segment (start 132.5238 100.33) (end 133.604 100.33) (width 0.3302) (layer F.Cu) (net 5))
 (segment (start 133.604 99.06) (end 123.698 99.06) (width 0.3302) (layer F.Cu) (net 6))
 (segment (start 123.698 96.52) (end 125.0442 96.52) (width 0.3302) (layer F.Cu) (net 7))
 (segment (start 125.0442 96.52) (end 126.3142 97.79) (width 0.3302) (layer F.Cu) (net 7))
 (segment (start 132.5238 97.79) (end 133.604 97.79) (width 0.3302) (layer F.Cu) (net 7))
 (segment (start 126.3142 97.79) (end 132.5238 97.79) (width 0.3302) (layer F.Cu) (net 7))
 (segment (start 139.004 101.6) (end 140.0842 101.6) (width 0.3302) (layer F.Cu) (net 8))
 (segment (start 140.0842 101.6) (end 141.3991 102.9149) (width 0.3302) (layer F.Cu) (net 8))
 (segment (start 141.3991 102.9149) (end 142.0195 102.9149) (width 0.3302) (layer F.Cu) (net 8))
 (segment (start 140.557402 100.625402) (end 141.930002 100.625402) (width 0.508) (layer F.Cu) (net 9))
 (segment (start 141.930002 100.625402) (end 142.0195 100.7149) (width 0.508) (layer F.Cu) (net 9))
 (segment (start 139.004 100.33) (end 140.262 100.33) (width 0.508) (layer F.Cu) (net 9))
 (segment (start 140.262 100.33) (end 140.557402 100.625402) (width 0.508) (layer F.Cu) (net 9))
 (segment (start 139.004 97.79) (end 140.262 97.79) (width 0.508) (layer F.Cu) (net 10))
 (segment (start 140.262 97.79) (end 140.6371 97.4149) (width 0.508) (layer F.Cu) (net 10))
 (segment (start 140.6371 97.4149) (end 142.0195 97.4149) (width 0.508) (layer F.Cu) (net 10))
 (segment (start 140.4664 99.06) (end 139.004 99.06) (width 0.508) (layer F.Cu) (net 11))
 (segment (start 142.0195 98.5149) (end 141.0115 98.5149) (width 0.508) (layer F.Cu) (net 11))
 (segment (start 141.0115 98.5149) (end 140.4664 99.06) (width 0.508) (layer F.Cu) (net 11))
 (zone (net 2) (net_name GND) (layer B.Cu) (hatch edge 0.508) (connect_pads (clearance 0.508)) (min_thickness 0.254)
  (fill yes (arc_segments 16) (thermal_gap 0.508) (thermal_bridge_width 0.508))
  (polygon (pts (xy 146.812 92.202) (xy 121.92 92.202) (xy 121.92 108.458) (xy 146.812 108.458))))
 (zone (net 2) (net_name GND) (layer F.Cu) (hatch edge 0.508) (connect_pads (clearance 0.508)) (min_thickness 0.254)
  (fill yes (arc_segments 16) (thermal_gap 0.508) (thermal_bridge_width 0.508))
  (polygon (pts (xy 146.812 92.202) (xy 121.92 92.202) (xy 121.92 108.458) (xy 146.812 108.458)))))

